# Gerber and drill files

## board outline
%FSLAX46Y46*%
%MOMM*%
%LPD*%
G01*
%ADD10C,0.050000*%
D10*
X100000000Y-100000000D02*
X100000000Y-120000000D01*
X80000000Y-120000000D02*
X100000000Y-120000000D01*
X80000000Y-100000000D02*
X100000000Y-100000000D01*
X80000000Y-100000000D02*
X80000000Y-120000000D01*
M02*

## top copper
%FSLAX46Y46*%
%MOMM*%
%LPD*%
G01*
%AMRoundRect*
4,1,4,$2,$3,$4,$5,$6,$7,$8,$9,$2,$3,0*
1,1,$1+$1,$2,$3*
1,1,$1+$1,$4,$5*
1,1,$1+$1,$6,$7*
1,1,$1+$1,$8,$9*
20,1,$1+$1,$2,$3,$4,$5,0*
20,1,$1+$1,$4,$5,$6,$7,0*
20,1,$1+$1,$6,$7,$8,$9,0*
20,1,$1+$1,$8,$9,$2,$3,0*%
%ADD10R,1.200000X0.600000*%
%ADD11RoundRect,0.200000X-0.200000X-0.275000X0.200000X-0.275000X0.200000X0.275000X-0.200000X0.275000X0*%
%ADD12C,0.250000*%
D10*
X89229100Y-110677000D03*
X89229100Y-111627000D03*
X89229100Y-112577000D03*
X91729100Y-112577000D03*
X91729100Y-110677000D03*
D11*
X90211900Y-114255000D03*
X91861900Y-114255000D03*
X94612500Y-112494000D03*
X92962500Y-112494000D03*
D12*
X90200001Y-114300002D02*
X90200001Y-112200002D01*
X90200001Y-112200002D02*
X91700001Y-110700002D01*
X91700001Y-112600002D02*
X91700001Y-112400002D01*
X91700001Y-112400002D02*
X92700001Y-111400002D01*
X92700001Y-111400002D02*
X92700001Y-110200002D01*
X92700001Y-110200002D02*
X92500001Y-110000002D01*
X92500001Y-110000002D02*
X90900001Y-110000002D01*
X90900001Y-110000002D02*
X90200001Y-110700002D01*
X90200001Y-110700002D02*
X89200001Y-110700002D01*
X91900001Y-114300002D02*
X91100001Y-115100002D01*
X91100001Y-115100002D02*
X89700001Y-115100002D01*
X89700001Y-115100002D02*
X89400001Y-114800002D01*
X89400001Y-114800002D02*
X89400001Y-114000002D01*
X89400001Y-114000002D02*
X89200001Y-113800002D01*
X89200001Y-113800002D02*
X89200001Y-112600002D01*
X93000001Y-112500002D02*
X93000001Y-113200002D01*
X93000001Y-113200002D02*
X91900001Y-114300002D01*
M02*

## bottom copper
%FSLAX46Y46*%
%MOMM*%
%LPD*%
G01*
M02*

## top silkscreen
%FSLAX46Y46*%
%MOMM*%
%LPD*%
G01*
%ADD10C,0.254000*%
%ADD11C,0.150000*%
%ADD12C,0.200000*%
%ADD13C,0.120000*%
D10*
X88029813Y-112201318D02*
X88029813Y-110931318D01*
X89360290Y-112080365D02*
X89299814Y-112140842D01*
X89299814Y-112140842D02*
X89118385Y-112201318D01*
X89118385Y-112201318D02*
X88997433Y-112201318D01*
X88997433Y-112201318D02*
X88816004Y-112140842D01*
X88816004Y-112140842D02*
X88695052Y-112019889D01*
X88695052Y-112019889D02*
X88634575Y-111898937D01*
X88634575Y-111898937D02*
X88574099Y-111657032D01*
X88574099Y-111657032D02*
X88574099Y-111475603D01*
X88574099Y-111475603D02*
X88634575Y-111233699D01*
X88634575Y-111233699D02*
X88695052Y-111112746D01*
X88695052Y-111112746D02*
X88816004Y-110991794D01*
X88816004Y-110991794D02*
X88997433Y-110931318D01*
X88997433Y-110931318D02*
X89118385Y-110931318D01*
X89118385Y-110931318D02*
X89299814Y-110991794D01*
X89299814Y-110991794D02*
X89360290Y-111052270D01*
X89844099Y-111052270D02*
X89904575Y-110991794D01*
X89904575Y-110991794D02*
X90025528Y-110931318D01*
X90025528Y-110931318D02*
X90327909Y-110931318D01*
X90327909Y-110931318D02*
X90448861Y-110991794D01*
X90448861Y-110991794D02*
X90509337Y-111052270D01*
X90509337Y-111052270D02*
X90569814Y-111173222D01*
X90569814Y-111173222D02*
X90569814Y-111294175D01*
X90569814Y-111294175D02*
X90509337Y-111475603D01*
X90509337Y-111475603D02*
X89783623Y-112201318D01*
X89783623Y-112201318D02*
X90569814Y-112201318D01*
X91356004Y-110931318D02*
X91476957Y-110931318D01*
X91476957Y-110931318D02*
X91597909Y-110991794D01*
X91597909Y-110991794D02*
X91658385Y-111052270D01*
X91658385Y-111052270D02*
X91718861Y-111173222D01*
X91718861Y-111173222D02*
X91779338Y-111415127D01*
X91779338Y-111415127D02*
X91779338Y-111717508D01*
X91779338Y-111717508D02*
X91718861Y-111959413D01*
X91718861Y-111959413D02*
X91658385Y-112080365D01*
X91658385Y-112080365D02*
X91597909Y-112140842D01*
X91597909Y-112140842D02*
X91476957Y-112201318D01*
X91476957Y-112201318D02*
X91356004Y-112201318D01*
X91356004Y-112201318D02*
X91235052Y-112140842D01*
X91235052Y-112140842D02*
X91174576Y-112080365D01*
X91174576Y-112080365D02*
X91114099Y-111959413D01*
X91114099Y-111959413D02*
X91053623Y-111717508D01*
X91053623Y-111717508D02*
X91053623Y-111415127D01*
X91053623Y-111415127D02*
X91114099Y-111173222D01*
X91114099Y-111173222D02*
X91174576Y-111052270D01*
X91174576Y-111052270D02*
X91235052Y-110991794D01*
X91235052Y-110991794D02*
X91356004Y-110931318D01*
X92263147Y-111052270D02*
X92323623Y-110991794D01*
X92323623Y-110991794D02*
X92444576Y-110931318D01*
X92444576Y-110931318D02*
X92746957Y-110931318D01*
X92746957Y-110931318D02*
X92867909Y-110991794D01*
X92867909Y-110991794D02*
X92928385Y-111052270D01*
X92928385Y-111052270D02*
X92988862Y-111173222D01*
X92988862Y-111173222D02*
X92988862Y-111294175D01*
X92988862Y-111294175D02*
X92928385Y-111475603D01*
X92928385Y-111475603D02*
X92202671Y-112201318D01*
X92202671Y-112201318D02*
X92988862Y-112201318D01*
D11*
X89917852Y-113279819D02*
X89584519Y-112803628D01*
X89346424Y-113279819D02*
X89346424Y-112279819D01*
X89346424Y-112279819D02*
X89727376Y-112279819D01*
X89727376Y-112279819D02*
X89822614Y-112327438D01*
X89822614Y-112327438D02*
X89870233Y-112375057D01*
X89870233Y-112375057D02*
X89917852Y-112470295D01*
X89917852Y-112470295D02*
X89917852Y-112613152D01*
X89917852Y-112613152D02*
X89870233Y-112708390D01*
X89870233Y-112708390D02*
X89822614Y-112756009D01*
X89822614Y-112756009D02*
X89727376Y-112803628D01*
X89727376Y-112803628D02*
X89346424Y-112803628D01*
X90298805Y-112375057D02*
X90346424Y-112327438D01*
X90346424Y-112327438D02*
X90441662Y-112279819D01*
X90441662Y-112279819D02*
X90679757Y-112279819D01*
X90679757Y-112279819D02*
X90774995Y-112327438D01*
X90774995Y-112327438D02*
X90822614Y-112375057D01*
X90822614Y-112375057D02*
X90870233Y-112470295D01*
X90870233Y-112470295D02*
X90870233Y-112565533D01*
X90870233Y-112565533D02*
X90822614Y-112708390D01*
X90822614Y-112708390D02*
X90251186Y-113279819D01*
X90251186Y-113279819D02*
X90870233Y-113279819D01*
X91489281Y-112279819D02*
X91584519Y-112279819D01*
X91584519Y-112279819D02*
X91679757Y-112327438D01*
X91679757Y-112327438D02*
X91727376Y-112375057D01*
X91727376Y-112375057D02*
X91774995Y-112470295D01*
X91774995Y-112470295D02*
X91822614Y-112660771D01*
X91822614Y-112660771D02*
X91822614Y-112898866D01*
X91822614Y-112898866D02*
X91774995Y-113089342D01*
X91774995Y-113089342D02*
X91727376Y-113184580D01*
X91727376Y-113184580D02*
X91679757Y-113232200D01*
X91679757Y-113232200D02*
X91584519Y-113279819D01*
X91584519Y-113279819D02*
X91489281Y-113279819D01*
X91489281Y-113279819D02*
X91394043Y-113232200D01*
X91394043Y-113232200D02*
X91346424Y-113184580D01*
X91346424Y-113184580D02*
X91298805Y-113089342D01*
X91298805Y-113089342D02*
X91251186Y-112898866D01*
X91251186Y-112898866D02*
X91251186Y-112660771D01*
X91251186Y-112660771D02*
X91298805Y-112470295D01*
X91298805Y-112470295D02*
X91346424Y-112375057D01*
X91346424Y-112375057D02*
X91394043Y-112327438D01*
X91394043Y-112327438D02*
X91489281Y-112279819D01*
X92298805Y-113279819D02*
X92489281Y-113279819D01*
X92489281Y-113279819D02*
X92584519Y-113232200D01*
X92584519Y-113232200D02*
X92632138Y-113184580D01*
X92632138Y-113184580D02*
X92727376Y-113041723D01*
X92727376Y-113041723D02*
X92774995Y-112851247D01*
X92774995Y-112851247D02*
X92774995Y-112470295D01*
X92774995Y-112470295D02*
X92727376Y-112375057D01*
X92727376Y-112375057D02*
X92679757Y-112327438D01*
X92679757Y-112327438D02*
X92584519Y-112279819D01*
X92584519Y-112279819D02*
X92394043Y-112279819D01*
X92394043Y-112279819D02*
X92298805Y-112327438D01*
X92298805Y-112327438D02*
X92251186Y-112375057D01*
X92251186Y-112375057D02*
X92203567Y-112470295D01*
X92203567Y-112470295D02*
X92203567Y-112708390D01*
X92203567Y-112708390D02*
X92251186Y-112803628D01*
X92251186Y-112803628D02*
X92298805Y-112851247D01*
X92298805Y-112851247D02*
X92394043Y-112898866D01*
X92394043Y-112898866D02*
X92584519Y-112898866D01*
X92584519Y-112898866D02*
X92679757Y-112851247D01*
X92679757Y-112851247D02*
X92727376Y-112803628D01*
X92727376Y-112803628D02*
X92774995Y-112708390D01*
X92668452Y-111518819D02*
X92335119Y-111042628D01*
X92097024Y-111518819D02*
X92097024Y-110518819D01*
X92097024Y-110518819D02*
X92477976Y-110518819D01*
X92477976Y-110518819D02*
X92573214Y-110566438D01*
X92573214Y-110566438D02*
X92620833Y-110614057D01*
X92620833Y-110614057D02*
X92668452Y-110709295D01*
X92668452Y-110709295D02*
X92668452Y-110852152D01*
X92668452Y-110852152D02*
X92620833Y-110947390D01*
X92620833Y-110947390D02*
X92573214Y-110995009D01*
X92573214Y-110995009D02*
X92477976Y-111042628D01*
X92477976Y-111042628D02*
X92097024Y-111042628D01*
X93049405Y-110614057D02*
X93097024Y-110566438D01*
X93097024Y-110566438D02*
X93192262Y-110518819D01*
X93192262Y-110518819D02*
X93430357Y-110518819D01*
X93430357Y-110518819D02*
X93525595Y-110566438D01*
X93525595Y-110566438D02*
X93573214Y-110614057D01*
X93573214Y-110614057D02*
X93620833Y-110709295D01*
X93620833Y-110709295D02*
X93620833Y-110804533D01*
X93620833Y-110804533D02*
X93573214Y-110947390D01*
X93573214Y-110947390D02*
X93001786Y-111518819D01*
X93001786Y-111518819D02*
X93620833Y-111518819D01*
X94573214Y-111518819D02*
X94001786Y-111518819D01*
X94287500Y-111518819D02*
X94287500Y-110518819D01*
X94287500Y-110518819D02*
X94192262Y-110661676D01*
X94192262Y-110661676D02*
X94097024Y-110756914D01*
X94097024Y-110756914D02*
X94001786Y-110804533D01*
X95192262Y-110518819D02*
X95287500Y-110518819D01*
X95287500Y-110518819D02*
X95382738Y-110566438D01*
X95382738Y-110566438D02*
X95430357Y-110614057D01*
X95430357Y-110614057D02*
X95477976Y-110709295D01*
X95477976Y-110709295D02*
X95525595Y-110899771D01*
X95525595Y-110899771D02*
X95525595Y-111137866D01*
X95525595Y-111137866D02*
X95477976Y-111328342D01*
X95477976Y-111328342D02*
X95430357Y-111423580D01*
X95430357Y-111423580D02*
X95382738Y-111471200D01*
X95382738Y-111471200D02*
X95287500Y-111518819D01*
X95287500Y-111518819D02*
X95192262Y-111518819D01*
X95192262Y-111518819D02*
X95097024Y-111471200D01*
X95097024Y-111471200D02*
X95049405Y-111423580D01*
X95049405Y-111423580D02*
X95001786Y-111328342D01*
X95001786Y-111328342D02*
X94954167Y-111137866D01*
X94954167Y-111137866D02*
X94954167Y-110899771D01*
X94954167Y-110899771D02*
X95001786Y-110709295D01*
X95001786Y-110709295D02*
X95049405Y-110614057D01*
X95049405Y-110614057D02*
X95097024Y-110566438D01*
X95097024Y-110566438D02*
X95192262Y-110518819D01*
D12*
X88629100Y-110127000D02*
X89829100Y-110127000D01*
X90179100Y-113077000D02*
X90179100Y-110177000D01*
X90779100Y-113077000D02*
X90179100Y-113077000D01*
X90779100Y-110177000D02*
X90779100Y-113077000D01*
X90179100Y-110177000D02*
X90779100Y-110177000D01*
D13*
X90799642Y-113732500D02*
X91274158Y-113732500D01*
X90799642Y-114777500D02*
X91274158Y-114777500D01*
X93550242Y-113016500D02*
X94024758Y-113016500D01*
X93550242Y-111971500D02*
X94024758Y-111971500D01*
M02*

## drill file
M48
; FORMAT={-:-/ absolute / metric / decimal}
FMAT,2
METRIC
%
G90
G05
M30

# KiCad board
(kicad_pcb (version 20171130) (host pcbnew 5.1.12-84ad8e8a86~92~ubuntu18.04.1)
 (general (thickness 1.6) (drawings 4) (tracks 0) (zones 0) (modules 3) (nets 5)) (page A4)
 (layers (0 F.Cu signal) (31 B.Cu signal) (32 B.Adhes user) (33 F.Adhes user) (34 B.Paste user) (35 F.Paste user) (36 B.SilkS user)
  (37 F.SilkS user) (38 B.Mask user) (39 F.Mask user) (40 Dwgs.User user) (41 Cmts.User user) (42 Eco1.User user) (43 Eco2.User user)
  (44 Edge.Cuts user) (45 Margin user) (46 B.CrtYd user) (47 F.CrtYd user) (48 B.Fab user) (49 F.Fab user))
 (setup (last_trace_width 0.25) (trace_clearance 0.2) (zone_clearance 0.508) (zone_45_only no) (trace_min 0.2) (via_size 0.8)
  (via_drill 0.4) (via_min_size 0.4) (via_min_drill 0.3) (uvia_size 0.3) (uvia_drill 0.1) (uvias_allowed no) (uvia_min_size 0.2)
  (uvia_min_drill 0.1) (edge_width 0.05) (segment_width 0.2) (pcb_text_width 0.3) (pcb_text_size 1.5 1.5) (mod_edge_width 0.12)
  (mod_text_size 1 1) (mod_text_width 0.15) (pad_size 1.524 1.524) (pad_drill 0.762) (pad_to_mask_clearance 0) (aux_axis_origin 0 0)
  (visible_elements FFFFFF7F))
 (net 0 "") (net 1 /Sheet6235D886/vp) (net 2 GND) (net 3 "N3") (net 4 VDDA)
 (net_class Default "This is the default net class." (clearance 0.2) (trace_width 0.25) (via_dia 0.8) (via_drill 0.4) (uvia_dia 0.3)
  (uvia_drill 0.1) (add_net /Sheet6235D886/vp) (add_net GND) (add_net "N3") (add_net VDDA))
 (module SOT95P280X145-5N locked (layer F.Cu) (at 90.479100 111.627000)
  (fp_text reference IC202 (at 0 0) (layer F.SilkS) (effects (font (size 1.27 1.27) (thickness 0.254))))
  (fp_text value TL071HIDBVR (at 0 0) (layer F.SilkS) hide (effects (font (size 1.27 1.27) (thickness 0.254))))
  (fp_line (start -1.85 -1.5) (end -0.65 -1.5) (layer F.SilkS) (width 0.2))
  (fp_line (start -0.3 1.45) (end -0.3 -1.45) (layer F.SilkS) (width 0.2))
  (fp_line (start 0.3 1.45) (end -0.3 1.45) (layer F.SilkS) (width 0.2))
  (fp_line (start 0.3 -1.45) (end 0.3 1.45) (layer F.SilkS) (width 0.2))
  (fp_line (start -0.3 -1.45) (end 0.3 -1.45) (layer F.SilkS) (width 0.2))
  (pad 1 smd rect (at -1.25 -0.95 90.000000) (size 0.6 1.2) (layers F.Cu F.Mask F.Paste) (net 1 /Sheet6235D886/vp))
  (pad 2 smd rect (at -1.25 0 90.000000) (size 0.6 1.2) (layers F.Cu F.Mask F.Paste) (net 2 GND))
  (pad 3 smd rect (at -1.25 0.95 90.000000) (size 0.6 1.2) (layers F.Cu F.Mask F.Paste) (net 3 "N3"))
  (pad 4 smd rect (at 1.25 0.95 90.000000) (size 0.6 1.2) (layers F.Cu F.Mask F.Paste) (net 1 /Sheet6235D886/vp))
  (pad 5 smd rect (at 1.25 -0.95 90.000000) (size 0.6 1.2) (layers F.Cu F.Mask F.Paste) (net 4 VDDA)))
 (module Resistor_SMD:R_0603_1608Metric (layer F.Cu) (at 91.036900 114.255000)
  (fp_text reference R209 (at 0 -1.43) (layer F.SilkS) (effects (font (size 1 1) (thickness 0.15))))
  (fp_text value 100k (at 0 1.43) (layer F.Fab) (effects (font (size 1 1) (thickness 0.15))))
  (fp_line (start -0.237258 -0.5225) (end 0.237258 -0.5225) (layer F.SilkS) (width 0.12))
  (fp_line (start -0.237258 0.5225) (end 0.237258 0.5225) (layer F.SilkS) (width 0.12))
  (pad 1 smd roundrect (at -0.825 0) (size 0.8 0.95) (layers F.Cu F.Mask F.Paste) (roundrect_rratio 0.25) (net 4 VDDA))
  (pad 2 smd roundrect (at 0.825 0) (size 0.8 0.95) (layers F.Cu F.Mask F.Paste) (roundrect_rratio 0.25) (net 3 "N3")))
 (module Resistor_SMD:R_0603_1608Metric (layer F.Cu) (at 93.787500 112.494000)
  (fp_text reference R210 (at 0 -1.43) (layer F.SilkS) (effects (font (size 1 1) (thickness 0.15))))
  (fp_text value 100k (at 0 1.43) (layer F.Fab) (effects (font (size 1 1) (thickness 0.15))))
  (fp_line (start -0.237258 0.5225) (end 0.237258 0.5225) (layer F.SilkS) (width 0.12))
  (fp_line (start -0.237258 -0.5225) (end 0.237258 -0.5225) (layer F.SilkS) (width 0.12))
  (pad 2 smd roundrect (at 0.825 0) (size 0.8 0.95) (layers F.Cu F.Mask F.Paste) (roundrect_rratio 0.25) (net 2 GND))
  (pad 1 smd roundrect (at -0.825 0) (size 0.8 0.95) (layers F.Cu F.Mask F.Paste) (roundrect_rratio 0.25) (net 3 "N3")))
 (gr_line (start 100 100) (end 100 120) (layer Edge.Cuts) (width 0.05))
 (gr_line (start 80 120) (end 100 120) (layer Edge.Cuts) (width 0.05))
 (gr_line (start 80 100) (end 100 100) (layer Edge.Cuts) (width 0.05))
 (gr_line (start 80 100) (end 80 120) (layer Edge.Cuts) (width 0.05))
 (segment (start 90.200001 114.300002) (end 90.200001 112.200002) (width 0.250000) (layer F.Cu) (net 4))
 (segment (start 90.200001 112.200002) (end 91.700001 110.700002) (width 0.250000) (layer F.Cu) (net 4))
 (segment (start 91.700001 112.600002) (end 91.700001 112.400002) (width 0.250000) (layer F.Cu) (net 1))
 (segment (start 91.700001 112.400002) (end 92.700001 111.400002) (width 0.250000) (layer F.Cu) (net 1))
 (segment (start 92.700001 111.400002) (end 92.700001 110.200002) (width 0.250000) (layer F.Cu) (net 1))
 (segment (start 92.700001 110.200002) (end 92.500001 110.000002) (width 0.250000) (layer F.Cu) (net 1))
 (segment (start 92.500001 110.000002) (end 90.900001 110.000002) (width 0.250000) (layer F.Cu) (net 1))
 (segment (start 90.900001 110.000002) (end 90.200001 110.700002) (width 0.250000) (layer F.Cu) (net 1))
 (segment (start 90.200001 110.700002) (end 89.200001 110.700002) (width 0.250000) (layer F.Cu) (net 1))
 (segment (start 91.900001 114.300002) (end 91.100001 115.100002) (width 0.250000) (layer F.Cu) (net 3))
 (segment (start 91.100001 115.100002) (end 89.700001 115.100002) (width 0.250000) (layer F.Cu) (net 3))
 (segment (start 89.700001 115.100002) (end 89.400001 114.800002) (width 0.250000) (layer F.Cu) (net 3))
 (segment (start 89.400001 114.800002) (end 89.400001 114.000002) (width 0.250000) (layer F.Cu) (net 3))
 (segment (start 89.400001 114.000002) (end 89.200001 113.800002) (width 0.250000) (layer F.Cu) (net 3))
 (segment (start 89.200001 113.800002) (end 89.200001 112.600002) (width 0.250000) (layer F.Cu) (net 3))
 (segment (start 93.000001 112.500002) (end 93.000001 113.200002) (width 0.250000) (layer F.Cu) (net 3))
 (segment (start 93.000001 113.200002) (end 91.900001 114.300002) (width 0.250000) (layer F.Cu) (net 3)))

